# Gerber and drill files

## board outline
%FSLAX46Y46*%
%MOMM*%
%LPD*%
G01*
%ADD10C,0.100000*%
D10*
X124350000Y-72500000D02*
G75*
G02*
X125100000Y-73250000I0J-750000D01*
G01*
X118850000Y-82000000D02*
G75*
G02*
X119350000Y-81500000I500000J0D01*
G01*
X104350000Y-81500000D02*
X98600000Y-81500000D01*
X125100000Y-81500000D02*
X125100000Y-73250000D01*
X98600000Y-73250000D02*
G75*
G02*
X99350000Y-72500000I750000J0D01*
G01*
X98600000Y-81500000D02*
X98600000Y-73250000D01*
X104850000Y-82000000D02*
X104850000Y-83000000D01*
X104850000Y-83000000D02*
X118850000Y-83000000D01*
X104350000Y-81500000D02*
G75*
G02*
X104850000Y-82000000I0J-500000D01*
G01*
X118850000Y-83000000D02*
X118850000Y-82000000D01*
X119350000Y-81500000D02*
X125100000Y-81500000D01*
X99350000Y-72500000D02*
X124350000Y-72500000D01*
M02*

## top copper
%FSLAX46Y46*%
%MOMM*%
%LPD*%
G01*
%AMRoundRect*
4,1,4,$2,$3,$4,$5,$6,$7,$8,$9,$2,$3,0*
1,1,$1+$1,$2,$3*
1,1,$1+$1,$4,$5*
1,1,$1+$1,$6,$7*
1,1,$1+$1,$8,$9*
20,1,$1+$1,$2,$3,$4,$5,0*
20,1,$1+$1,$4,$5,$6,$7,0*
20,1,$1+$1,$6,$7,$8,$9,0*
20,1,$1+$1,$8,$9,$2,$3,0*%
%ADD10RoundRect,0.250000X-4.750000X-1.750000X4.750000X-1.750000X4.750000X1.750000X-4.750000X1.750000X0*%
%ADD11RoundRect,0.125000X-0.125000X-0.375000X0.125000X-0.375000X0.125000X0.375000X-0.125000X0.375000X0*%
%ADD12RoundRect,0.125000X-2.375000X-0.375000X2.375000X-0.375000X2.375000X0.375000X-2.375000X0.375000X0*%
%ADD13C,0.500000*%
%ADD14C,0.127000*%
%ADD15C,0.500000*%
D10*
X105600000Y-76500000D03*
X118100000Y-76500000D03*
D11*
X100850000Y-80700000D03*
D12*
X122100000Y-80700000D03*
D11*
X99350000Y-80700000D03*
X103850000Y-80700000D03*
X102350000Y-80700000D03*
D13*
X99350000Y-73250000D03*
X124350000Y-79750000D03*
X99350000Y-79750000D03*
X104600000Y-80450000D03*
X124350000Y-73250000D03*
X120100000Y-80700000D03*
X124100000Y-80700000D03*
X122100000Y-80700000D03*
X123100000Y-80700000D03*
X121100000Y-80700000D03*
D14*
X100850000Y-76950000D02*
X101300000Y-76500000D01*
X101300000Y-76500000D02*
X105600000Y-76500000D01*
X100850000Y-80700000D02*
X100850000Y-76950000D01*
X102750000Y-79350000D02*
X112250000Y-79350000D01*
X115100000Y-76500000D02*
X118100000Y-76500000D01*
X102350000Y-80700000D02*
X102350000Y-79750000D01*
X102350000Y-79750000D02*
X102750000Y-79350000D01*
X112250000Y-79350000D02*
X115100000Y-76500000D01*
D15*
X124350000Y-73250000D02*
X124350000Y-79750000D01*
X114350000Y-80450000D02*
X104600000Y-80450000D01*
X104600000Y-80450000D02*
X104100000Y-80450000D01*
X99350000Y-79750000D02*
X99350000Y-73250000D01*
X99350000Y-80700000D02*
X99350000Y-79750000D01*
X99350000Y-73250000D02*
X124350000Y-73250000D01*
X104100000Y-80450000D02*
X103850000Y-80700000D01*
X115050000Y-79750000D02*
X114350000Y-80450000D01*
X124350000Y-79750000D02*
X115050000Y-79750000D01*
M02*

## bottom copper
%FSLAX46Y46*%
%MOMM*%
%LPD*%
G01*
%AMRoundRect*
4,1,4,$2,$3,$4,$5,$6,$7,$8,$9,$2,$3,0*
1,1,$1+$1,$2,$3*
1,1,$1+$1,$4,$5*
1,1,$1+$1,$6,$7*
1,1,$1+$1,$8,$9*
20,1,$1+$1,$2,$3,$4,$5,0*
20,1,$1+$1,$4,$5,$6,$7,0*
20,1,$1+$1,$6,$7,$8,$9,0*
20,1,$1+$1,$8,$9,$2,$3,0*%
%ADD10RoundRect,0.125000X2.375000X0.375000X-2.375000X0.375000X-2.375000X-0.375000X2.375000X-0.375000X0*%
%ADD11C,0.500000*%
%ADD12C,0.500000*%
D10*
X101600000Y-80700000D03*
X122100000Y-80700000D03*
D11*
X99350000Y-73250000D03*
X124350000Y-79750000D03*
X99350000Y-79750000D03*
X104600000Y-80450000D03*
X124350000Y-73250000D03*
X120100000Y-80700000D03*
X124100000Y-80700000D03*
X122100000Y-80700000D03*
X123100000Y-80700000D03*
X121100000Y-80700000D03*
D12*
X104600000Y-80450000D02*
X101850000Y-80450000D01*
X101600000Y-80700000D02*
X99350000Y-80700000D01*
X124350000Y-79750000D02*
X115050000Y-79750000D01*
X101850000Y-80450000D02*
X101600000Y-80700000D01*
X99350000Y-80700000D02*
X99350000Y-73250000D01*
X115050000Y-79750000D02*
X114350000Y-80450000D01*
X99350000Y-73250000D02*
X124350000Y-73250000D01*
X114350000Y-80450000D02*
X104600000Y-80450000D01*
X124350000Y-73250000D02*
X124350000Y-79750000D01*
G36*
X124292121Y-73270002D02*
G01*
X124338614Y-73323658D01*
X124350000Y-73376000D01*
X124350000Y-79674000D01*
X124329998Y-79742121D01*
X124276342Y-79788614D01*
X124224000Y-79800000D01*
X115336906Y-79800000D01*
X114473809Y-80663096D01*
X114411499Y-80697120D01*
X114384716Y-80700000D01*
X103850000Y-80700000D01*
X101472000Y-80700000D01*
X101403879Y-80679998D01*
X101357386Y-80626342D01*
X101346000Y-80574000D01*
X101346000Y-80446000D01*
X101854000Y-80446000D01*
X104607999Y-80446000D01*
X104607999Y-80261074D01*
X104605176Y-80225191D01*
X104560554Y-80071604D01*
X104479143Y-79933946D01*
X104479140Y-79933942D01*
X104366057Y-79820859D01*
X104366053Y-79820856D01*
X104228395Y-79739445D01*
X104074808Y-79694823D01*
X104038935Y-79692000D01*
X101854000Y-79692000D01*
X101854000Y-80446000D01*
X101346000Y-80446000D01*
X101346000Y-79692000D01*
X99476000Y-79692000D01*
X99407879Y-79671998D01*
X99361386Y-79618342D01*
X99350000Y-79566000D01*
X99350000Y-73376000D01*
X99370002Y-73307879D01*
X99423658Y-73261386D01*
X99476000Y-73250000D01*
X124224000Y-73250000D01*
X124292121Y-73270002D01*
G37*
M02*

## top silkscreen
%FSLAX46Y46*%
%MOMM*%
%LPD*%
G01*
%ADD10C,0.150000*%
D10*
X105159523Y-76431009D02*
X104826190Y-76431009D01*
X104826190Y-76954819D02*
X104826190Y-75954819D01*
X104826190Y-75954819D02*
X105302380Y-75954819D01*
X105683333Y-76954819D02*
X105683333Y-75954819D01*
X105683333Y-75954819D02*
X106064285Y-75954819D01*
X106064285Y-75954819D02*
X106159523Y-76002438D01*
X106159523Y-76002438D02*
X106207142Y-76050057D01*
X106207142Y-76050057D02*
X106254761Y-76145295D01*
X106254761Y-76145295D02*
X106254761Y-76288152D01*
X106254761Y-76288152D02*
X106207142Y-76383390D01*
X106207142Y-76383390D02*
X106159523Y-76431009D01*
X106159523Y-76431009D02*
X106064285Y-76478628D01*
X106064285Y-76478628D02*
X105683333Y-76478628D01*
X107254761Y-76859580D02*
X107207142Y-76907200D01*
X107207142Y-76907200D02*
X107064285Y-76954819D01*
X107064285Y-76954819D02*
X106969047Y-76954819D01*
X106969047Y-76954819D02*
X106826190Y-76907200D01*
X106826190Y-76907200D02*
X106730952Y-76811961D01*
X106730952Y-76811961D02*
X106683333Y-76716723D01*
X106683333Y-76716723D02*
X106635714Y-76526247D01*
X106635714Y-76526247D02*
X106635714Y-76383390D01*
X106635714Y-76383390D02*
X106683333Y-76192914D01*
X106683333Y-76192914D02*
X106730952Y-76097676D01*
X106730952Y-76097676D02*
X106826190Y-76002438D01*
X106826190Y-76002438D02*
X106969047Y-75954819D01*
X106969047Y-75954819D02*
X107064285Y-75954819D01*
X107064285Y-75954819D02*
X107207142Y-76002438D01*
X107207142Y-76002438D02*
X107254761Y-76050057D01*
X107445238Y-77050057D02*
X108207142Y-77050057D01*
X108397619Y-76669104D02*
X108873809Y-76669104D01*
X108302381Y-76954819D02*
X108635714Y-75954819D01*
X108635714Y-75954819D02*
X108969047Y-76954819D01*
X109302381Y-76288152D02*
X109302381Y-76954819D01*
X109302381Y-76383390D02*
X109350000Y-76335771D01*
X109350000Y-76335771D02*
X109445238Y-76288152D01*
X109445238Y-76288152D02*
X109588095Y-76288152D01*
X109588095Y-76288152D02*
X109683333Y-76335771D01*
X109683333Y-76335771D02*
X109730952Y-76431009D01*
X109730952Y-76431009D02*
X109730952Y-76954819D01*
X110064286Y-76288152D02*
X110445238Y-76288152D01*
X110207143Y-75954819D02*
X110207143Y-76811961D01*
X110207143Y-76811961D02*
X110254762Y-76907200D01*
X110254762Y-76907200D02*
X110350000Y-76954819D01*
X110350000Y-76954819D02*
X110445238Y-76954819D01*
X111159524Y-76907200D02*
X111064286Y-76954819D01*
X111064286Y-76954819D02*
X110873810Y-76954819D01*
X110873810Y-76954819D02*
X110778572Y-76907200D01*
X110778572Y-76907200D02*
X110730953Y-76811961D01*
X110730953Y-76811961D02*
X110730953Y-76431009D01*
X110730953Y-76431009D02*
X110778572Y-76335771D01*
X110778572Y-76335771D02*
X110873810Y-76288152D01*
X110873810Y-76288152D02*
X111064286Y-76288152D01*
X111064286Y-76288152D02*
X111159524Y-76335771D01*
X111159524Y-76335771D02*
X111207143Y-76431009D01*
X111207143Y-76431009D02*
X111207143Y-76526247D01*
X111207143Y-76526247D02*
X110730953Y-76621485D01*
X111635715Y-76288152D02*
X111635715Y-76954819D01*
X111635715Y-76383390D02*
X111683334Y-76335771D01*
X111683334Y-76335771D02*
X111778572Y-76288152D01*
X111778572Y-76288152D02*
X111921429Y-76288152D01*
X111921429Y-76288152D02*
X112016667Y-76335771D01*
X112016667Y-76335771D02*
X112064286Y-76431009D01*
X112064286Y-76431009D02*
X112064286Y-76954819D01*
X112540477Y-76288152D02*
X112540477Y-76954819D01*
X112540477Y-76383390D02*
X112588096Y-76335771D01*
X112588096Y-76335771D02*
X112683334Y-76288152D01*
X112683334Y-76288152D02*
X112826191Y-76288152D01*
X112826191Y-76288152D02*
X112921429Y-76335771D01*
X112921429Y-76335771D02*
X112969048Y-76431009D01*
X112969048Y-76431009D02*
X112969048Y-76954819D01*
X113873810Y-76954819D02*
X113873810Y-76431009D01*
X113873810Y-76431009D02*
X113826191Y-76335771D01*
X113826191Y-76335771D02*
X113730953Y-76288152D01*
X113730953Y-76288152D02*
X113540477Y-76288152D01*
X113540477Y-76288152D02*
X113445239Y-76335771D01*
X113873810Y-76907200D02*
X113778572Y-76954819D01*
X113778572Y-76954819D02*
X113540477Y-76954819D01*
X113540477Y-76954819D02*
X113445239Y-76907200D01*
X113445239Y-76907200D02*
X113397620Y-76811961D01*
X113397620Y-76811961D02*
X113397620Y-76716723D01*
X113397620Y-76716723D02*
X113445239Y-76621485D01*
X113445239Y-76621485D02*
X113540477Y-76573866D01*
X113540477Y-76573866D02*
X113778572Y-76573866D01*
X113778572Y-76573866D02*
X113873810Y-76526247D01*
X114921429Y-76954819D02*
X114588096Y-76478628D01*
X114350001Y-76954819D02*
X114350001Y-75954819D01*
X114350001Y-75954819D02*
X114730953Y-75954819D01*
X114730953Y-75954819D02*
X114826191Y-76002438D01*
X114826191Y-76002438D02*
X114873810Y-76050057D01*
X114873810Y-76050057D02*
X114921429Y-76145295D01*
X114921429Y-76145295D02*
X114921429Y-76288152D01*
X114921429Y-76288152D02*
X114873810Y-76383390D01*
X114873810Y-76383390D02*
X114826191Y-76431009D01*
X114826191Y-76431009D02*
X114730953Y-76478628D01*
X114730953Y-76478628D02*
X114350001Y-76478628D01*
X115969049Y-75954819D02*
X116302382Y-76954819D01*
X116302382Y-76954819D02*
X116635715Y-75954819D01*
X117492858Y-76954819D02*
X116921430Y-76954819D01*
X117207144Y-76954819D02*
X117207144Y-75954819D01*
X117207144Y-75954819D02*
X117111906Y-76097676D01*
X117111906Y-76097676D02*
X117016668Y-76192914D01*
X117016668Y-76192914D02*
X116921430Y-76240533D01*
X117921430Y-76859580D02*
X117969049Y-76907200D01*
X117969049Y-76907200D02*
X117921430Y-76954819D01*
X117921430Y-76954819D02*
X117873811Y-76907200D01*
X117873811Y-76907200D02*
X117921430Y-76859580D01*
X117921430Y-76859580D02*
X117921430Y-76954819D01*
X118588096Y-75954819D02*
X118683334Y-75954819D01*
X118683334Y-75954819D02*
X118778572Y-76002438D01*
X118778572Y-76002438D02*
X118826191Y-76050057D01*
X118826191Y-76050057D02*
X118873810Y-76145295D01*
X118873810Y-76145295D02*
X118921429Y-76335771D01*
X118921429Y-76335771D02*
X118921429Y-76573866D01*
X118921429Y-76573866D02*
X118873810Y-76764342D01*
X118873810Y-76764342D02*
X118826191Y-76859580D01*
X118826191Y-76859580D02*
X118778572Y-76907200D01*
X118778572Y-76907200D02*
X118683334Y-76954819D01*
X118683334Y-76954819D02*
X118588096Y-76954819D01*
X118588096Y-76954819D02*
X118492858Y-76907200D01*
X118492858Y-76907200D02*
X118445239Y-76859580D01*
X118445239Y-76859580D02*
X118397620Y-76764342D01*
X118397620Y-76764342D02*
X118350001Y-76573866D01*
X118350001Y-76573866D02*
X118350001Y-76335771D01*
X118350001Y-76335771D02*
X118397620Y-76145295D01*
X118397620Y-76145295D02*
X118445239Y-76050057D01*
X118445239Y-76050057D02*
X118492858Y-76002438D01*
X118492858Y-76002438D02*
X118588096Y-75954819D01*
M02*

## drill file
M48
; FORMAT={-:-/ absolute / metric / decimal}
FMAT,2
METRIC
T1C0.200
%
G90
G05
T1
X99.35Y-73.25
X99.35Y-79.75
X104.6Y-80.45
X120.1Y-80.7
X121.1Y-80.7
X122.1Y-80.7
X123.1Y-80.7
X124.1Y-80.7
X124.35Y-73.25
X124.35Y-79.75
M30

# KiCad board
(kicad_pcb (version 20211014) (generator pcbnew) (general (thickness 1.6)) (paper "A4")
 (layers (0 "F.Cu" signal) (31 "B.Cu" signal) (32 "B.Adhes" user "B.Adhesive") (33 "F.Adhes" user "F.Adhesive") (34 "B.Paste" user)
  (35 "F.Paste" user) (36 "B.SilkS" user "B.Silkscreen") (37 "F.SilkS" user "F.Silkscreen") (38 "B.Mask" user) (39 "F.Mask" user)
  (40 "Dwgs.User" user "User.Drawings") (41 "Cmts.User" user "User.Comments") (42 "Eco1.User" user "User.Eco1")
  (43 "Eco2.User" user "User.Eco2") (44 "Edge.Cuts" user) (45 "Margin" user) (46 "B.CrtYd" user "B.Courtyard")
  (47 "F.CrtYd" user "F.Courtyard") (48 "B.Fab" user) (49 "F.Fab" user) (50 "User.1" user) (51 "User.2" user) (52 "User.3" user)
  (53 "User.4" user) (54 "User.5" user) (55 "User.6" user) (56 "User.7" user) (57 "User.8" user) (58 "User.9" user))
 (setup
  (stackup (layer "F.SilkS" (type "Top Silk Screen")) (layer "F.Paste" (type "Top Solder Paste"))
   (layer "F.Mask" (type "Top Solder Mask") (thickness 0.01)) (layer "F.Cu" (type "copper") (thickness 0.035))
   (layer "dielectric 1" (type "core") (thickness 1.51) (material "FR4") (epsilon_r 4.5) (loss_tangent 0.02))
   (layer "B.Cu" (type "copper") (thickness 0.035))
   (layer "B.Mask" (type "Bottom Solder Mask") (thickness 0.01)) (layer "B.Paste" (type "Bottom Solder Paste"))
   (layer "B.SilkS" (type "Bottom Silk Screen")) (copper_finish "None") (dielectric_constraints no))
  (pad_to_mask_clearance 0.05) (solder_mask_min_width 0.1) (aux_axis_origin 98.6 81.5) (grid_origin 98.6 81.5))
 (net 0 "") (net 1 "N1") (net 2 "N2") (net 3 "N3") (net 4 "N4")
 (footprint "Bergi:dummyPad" (layer "F.Cu") (at 105.6 76.5)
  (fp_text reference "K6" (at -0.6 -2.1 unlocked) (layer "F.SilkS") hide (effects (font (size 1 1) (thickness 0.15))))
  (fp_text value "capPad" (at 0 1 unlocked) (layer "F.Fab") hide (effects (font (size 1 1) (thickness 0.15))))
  (pad "1" smd roundrect (at 0 0) (size 10 4) (layers "F.Cu") (roundrect_rratio 0.0625) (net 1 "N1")))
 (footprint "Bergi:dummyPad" (layer "F.Cu") (at 118.1 76.5)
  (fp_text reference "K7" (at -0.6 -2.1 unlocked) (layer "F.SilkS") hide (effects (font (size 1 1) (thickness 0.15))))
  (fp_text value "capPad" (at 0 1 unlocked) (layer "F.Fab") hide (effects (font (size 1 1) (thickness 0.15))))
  (pad "1" smd roundrect (at 0 0) (size 10 4) (layers "F.Cu") (roundrect_rratio 0.0625) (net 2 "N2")))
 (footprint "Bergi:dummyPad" (layer "F.Cu") (at 100.85 80.7)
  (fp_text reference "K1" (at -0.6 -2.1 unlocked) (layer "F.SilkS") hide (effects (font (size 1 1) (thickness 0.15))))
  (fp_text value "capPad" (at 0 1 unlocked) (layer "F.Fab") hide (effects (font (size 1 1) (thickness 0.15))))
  (pad "1" smd roundrect (at 0 0) (size 0.5 1) (layers "F.Cu" "F.Mask") (roundrect_rratio 0.25) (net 1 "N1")))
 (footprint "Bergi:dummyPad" (layer "F.Cu") (at 122.1 80.7)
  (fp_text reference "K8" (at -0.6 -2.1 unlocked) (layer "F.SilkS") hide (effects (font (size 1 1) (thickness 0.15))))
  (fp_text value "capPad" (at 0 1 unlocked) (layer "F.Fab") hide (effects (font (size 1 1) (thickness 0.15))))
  (pad "1" smd roundrect (at 0 0) (size 5 1) (layers "F.Cu" "F.Mask") (roundrect_rratio 0.125) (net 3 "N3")))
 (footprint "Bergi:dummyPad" (layer "F.Cu") (at 99.35 80.7)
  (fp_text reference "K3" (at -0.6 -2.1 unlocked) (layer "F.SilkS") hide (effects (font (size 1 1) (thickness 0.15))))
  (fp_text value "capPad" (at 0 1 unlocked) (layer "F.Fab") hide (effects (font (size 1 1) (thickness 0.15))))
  (pad "1" smd roundrect (at 0 0) (size 0.5 1) (layers "F.Cu" "F.Mask") (roundrect_rratio 0.25) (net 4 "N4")))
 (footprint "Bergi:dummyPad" (layer "F.Cu") (at 103.85 80.7)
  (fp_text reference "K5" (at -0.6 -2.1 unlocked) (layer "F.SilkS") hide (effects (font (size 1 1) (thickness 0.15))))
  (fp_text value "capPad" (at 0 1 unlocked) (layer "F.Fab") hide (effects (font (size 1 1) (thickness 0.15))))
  (pad "1" smd roundrect (at 0 0) (size 0.5 1) (layers "F.Cu" "F.Mask") (roundrect_rratio 0.25) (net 4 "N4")))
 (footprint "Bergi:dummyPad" (layer "F.Cu") (at 102.35 80.7)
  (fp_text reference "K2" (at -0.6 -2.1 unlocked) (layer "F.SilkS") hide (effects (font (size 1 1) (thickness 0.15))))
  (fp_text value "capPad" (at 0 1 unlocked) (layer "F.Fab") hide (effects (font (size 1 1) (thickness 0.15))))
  (pad "1" smd roundrect (at 0 0) (size 0.5 1) (layers "F.Cu" "F.Mask") (roundrect_rratio 0.25) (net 2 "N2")))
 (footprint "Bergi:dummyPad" (layer "B.Cu") (at 101.6 80.7 180)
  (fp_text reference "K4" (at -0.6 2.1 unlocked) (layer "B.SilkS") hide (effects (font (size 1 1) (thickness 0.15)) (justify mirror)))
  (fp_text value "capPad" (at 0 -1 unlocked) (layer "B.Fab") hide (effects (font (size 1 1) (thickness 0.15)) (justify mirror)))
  (pad "1" smd roundrect (at 0 0 180) (size 5 1) (layers "B.Cu" "B.Mask") (roundrect_rratio 0.125) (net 4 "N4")))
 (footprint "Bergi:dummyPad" (layer "B.Cu") (at 122.1 80.7 180)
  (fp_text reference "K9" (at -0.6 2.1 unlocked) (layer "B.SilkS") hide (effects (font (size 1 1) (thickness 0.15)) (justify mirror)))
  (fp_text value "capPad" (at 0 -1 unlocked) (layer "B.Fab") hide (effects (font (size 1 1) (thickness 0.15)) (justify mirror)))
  (pad "1" smd roundrect (at 0 0 180) (size 5 1) (layers "B.Cu" "B.Mask") (roundrect_rratio 0.125) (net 3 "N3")))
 (gr_arc (start 124.35 72.5) (mid 124.88033 72.71967) (end 125.1 73.25) (layer "Edge.Cuts") (width 0.1))
 (gr_arc (start 118.85 82) (mid 118.996447 81.646447) (end 119.35 81.5) (layer "Edge.Cuts") (width 0.1))
 (gr_line (start 104.35 81.5) (end 98.6 81.5) (layer "Edge.Cuts") (width 0.1))
 (gr_line (start 125.1 81.5) (end 125.1 73.25) (layer "Edge.Cuts") (width 0.1))
 (gr_arc (start 98.6 73.25) (mid 98.81967 72.71967) (end 99.35 72.5) (layer "Edge.Cuts") (width 0.1))
 (gr_line (start 98.6 81.5) (end 98.6 73.25) (layer "Edge.Cuts") (width 0.1))
 (gr_line (start 104.85 82) (end 104.85 83) (layer "Edge.Cuts") (width 0.1))
 (gr_line (start 104.85 83) (end 118.85 83) (layer "Edge.Cuts") (width 0.1))
 (gr_arc (start 104.35 81.5) (mid 104.703553 81.646447) (end 104.85 82) (layer "Edge.Cuts") (width 0.1))
 (gr_line (start 118.85 83) (end 118.85 82) (layer "Edge.Cuts") (width 0.1))
 (gr_line (start 119.35 81.5) (end 125.1 81.5) (layer "Edge.Cuts") (width 0.1))
 (gr_line (start 99.35 72.5) (end 124.35 72.5) (layer "Edge.Cuts") (width 0.1))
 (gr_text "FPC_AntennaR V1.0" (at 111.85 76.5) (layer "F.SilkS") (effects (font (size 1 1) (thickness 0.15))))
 (segment (start 100.85 76.95) (end 101.3 76.5) (width 0.127) (layer "F.Cu") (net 1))
 (segment (start 101.3 76.5) (end 105.6 76.5) (width 0.127) (layer "F.Cu") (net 1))
 (segment (start 100.85 80.7) (end 100.85 76.95) (width 0.127) (layer "F.Cu") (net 1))
 (segment (start 102.75 79.35) (end 112.25 79.35) (width 0.127) (layer "F.Cu") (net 2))
 (segment (start 115.1 76.5) (end 118.1 76.5) (width 0.127) (layer "F.Cu") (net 2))
 (segment (start 102.35 80.7) (end 102.35 79.75) (width 0.127) (layer "F.Cu") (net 2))
 (segment (start 102.35 79.75) (end 102.75 79.35) (width 0.127) (layer "F.Cu") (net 2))
 (segment (start 112.25 79.35) (end 115.1 76.5) (width 0.127) (layer "F.Cu") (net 2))
 (segment (start 124.35 73.25) (end 124.35 79.75) (width 0.5) (layer "F.Cu") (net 4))
 (segment (start 114.35 80.45) (end 104.6 80.45) (width 0.5) (layer "F.Cu") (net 4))
 (segment (start 104.6 80.45) (end 104.1 80.45) (width 0.5) (layer "F.Cu") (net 4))
 (segment (start 99.35 79.75) (end 99.35 73.25) (width 0.5) (layer "F.Cu") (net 4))
 (segment (start 99.35 80.7) (end 99.35 79.75) (width 0.5) (layer "F.Cu") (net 4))
 (segment (start 99.35 73.25) (end 124.35 73.25) (width 0.5) (layer "F.Cu") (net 4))
 (segment (start 104.1 80.45) (end 103.85 80.7) (width 0.5) (layer "F.Cu") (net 4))
 (segment (start 115.05 79.75) (end 114.35 80.45) (width 0.5) (layer "F.Cu") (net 4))
 (segment (start 124.35 79.75) (end 115.05 79.75) (width 0.5) (layer "F.Cu") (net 4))
 (via (at 99.35 73.25) (size 0.5) (drill 0.2) (layers "F.Cu" "B.Cu") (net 4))
 (via (at 124.35 79.75) (size 0.5) (drill 0.2) (layers "F.Cu" "B.Cu") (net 4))
 (via (at 99.35 79.75) (size 0.5) (drill 0.2) (layers "F.Cu" "B.Cu") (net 4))
 (via (at 104.6 80.45) (size 0.5) (drill 0.2) (layers "F.Cu" "B.Cu") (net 4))
 (via (at 124.35 73.25) (size 0.5) (drill 0.2) (layers "F.Cu" "B.Cu") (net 4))
 (segment (start 104.6 80.45) (end 101.85 80.45) (width 0.5) (layer "B.Cu") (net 4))
 (segment (start 101.6 80.7) (end 99.35 80.7) (width 0.5) (layer "B.Cu") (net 4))
 (segment (start 124.35 79.75) (end 115.05 79.75) (width 0.5) (layer "B.Cu") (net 4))
 (segment (start 101.85 80.45) (end 101.6 80.7) (width 0.5) (layer "B.Cu") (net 4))
 (segment (start 99.35 80.7) (end 99.35 73.25) (width 0.5) (layer "B.Cu") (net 4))
 (segment (start 115.05 79.75) (end 114.35 80.45) (width 0.5) (layer "B.Cu") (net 4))
 (segment (start 99.35 73.25) (end 124.35 73.25) (width 0.5) (layer "B.Cu") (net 4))
 (segment (start 114.35 80.45) (end 104.6 80.45) (width 0.5) (layer "B.Cu") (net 4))
 (segment (start 124.35 73.25) (end 124.35 79.75) (width 0.5) (layer "B.Cu") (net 4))
 (via (at 120.1 80.7) (size 0.5) (drill 0.2) (layers "F.Cu" "B.Cu") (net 3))
 (via (at 124.1 80.7) (size 0.5) (drill 0.2) (layers "F.Cu" "B.Cu") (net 3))
 (via (at 122.1 80.7) (size 0.5) (drill 0.2) (layers "F.Cu" "B.Cu") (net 3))
 (via (at 123.1 80.7) (size 0.5) (drill 0.2) (layers "F.Cu" "B.Cu") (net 3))
 (via (at 121.1 80.7) (size 0.5) (drill 0.2) (layers "F.Cu" "B.Cu") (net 3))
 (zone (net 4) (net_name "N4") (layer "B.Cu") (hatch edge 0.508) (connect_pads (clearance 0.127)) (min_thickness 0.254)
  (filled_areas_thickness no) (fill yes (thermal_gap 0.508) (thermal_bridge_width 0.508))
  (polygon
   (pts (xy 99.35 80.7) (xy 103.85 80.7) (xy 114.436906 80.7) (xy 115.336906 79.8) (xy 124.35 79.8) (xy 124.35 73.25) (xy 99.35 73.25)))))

